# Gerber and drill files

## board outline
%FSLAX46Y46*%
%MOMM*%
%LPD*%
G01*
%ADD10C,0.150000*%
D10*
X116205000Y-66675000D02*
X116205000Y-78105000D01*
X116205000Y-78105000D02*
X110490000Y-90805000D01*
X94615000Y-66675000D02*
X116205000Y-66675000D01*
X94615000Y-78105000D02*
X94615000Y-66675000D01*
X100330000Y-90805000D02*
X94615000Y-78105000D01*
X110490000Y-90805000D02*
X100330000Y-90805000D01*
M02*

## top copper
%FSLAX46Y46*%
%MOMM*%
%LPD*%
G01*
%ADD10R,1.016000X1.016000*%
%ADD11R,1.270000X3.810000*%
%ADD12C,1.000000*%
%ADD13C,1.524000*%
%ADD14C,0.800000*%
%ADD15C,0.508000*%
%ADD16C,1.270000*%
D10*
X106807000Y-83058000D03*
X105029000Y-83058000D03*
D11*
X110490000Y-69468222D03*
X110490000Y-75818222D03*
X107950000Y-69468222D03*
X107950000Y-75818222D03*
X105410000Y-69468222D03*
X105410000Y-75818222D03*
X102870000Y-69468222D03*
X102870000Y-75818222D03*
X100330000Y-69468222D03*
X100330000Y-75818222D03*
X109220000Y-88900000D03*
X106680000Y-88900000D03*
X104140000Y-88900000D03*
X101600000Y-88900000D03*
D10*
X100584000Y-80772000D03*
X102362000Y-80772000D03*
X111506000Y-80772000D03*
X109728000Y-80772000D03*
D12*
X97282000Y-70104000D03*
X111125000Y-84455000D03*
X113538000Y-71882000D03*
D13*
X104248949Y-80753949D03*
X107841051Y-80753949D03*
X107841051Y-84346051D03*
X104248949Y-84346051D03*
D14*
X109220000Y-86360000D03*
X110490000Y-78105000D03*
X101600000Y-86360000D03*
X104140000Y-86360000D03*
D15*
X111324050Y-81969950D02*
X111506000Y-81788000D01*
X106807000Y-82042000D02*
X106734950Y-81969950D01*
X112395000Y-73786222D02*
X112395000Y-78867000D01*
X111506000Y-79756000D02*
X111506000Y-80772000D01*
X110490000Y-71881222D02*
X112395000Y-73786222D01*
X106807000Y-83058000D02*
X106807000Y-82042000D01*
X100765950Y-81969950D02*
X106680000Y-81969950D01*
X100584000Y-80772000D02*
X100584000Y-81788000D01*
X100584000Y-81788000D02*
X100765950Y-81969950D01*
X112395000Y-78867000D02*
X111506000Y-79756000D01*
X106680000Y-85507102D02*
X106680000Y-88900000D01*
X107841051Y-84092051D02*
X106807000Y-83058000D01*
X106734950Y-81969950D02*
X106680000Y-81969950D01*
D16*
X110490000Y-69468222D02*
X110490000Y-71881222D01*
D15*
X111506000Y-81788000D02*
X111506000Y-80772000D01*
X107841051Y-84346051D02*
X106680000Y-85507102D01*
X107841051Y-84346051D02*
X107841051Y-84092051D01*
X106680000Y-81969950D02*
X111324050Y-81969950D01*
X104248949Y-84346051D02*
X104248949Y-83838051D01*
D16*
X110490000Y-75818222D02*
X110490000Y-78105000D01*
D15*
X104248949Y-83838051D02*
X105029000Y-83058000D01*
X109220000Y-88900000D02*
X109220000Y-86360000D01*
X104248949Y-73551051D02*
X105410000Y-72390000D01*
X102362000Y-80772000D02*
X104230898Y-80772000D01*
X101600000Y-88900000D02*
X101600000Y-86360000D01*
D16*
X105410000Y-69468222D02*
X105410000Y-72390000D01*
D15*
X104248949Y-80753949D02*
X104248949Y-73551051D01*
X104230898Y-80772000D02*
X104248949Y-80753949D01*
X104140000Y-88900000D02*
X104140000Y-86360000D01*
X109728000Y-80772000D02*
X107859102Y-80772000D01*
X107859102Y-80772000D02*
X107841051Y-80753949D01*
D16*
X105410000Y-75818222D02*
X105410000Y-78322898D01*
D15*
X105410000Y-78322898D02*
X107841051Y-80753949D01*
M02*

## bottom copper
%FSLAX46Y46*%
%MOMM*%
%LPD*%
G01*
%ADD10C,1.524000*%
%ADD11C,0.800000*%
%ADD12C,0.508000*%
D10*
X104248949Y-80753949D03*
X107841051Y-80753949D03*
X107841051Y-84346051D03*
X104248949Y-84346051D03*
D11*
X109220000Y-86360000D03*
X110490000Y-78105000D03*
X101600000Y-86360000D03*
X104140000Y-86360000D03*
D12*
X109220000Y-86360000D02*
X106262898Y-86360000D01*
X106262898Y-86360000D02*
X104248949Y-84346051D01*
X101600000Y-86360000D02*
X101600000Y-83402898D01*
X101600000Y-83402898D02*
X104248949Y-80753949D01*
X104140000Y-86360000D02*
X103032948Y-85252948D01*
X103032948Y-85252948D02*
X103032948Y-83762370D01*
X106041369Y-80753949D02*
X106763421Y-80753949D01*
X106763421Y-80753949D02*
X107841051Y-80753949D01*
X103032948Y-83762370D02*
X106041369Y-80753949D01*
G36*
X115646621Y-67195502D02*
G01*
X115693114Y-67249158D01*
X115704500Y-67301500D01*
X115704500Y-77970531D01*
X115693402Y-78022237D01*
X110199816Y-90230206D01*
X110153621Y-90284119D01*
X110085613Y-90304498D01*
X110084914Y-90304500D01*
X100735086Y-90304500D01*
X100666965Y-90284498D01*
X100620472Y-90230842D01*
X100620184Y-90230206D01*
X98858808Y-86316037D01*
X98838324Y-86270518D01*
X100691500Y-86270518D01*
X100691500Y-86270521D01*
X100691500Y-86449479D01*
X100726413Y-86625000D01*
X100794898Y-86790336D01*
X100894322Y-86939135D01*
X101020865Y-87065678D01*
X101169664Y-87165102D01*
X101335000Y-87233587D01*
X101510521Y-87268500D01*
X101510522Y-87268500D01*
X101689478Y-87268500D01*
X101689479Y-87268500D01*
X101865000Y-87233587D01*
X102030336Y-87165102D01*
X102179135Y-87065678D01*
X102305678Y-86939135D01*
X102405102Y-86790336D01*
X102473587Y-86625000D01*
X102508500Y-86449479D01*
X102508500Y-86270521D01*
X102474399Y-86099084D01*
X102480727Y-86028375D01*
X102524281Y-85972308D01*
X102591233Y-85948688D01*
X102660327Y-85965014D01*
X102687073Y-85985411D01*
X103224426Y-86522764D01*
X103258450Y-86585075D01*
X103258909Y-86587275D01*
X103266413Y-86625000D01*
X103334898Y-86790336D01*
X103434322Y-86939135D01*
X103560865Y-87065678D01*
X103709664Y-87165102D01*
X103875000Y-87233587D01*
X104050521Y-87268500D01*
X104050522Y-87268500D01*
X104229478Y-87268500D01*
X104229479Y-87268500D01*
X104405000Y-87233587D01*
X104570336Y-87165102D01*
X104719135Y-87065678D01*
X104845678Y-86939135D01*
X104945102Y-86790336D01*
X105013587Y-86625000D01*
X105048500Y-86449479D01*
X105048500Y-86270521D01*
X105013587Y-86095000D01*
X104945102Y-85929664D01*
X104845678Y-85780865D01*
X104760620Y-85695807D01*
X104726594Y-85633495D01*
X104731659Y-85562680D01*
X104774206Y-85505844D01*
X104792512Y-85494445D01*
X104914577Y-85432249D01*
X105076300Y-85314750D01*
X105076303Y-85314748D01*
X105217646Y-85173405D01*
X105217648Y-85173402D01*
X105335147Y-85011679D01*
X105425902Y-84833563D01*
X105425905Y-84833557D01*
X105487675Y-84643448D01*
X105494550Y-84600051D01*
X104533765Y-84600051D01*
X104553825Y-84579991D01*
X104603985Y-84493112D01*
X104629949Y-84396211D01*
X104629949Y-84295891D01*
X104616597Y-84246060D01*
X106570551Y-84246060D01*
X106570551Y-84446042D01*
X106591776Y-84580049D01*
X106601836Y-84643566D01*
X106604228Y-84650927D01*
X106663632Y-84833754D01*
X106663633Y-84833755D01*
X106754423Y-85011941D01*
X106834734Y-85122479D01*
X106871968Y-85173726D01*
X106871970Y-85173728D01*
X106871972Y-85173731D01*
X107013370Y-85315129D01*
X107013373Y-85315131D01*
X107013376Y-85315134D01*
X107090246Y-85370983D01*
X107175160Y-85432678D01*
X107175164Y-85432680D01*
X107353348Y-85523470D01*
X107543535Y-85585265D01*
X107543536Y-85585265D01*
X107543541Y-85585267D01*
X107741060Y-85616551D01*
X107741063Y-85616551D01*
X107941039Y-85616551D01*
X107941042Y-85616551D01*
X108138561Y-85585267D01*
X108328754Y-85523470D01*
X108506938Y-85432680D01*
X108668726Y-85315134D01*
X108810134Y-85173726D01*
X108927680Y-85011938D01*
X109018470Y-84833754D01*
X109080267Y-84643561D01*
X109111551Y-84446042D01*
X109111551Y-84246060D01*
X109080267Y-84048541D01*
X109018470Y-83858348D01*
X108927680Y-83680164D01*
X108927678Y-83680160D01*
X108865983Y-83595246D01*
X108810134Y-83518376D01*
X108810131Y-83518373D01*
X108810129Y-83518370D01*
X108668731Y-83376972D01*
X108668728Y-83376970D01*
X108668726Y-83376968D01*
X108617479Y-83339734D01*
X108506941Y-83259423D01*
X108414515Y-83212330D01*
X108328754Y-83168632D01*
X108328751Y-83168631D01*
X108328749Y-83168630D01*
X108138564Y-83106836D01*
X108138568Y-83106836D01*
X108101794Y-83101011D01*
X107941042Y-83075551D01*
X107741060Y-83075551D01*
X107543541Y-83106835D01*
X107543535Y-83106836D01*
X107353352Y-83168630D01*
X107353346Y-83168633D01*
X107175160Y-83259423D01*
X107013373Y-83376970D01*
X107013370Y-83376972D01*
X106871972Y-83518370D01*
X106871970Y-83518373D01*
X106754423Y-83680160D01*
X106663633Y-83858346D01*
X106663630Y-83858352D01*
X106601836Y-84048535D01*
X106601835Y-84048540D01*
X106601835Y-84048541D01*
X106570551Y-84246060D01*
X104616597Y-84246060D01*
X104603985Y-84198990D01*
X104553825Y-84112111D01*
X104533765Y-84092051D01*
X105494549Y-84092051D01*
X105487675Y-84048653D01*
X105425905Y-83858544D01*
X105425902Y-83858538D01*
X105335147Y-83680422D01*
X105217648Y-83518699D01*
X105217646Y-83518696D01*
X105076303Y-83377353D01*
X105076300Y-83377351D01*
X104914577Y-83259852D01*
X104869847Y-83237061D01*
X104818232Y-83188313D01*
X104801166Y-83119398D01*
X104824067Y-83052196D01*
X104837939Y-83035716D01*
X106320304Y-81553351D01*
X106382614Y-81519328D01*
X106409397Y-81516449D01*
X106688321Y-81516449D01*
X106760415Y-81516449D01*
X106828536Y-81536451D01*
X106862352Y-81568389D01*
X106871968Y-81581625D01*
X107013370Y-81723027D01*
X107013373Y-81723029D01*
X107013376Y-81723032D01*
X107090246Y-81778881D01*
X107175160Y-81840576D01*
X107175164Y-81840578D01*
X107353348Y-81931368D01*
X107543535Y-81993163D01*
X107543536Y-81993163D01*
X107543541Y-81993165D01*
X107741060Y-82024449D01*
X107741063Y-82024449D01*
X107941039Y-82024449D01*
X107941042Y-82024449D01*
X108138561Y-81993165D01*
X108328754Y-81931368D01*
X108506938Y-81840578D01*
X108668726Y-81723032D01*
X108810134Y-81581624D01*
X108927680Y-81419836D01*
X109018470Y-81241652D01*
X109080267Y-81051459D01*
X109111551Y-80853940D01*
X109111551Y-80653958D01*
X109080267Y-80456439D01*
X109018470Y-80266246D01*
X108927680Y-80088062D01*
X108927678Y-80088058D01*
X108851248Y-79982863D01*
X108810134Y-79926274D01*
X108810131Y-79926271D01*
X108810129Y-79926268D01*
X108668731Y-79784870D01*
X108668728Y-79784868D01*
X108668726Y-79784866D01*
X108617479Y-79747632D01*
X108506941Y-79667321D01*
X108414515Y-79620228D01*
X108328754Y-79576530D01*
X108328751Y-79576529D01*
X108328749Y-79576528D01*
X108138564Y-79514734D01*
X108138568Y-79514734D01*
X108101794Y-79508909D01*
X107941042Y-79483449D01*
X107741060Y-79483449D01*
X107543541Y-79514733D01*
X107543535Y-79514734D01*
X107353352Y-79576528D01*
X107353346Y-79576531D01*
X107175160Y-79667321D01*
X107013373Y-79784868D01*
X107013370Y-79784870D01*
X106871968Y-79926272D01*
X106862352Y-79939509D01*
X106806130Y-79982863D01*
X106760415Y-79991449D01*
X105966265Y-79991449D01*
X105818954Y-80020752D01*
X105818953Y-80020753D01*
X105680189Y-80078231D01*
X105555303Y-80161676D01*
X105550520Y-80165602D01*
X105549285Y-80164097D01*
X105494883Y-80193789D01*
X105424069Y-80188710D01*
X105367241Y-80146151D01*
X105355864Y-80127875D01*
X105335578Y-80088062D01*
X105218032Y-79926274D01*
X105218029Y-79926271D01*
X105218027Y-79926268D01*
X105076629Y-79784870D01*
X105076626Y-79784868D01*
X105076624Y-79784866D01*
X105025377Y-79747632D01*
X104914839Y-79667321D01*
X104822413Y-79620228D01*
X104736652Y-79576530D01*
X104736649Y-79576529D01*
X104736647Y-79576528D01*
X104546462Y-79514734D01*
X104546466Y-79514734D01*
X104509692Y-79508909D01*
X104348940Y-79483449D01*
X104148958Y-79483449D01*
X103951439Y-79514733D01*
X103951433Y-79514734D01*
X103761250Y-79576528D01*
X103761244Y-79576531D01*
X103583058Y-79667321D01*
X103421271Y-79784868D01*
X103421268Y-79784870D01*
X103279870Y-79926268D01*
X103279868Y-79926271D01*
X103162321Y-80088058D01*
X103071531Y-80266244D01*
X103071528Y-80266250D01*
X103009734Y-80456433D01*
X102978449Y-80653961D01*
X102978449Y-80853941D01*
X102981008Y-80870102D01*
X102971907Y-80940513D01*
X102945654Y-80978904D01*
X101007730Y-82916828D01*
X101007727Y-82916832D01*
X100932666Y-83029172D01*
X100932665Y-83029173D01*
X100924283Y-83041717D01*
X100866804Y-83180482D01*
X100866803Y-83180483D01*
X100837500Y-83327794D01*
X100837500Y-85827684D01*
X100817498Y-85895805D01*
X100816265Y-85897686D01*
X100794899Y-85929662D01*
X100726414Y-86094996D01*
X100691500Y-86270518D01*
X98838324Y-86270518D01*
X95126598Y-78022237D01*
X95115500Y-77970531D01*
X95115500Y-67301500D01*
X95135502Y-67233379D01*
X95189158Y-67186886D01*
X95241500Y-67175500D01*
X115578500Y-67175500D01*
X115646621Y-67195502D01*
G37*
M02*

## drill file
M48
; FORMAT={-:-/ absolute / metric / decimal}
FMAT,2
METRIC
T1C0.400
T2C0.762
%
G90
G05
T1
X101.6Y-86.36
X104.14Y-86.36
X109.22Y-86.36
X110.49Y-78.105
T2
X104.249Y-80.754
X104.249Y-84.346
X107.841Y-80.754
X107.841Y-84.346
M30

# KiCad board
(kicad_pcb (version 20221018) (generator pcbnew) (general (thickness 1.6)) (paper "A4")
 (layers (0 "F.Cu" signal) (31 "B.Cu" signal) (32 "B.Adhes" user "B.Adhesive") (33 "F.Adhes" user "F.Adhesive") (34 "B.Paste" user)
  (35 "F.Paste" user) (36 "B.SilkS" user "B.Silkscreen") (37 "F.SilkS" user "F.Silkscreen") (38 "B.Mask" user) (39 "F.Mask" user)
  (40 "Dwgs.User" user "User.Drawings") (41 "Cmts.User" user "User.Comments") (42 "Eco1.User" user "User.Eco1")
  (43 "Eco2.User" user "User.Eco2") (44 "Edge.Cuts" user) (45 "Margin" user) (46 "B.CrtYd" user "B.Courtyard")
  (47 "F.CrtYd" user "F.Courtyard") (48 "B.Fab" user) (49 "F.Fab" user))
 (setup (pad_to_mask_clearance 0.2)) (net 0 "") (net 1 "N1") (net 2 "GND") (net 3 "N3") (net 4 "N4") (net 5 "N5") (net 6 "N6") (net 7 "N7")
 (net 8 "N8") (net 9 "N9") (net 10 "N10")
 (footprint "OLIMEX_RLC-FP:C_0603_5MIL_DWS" (layer "F.Cu") (at 105.918 83.058 180)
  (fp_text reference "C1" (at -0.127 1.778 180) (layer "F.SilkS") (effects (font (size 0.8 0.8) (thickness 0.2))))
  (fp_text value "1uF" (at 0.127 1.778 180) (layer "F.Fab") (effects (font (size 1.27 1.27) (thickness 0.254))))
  (pad "1" smd rect (at -0.889 0 180) (size 1.016 1.016) (layers "F.Cu" "F.Paste" "F.Mask") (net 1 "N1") (solder_mask_margin 0.0508)
   (clearance 0.0508))
  (pad "2" smd rect (at 0.889 0 180) (size 1.016 1.016) (layers "F.Cu" "F.Paste" "F.Mask") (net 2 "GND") (solder_mask_margin 0.0508)
   (clearance 0.0508)))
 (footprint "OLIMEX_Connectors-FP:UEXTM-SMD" (layer "F.Cu") (at 105.41 72.643222)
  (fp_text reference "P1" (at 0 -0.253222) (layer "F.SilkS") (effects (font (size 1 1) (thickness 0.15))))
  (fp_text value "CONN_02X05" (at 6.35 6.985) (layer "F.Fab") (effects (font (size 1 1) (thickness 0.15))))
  (pad "1" smd rect (at 5.08 -3.175) (size 1.27 3.81) (layers "F.Cu" "F.Paste" "F.Mask") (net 1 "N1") (solder_mask_margin 0.0508)
   (solder_paste_margin -0.0508) (clearance 0.0508))
  (pad "2" smd rect (at 5.08 3.175) (size 1.27 3.81) (layers "F.Cu" "F.Paste" "F.Mask") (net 2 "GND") (solder_mask_margin 0.0508)
   (solder_paste_margin -0.0508) (clearance 0.0508))
  (pad "3" smd rect (at 2.54 -3.175) (size 1.27 3.81) (layers "F.Cu" "F.Paste" "F.Mask") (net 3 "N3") (solder_mask_margin 0.0508)
   (solder_paste_margin -0.0508) (clearance 0.0508))
  (pad "4" smd rect (at 2.54 3.175) (size 1.27 3.81) (layers "F.Cu" "F.Paste" "F.Mask") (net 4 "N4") (solder_mask_margin 0.0508)
   (solder_paste_margin -0.0508) (clearance 0.0508))
  (pad "5" smd rect (at 0 -3.175) (size 1.27 3.81) (layers "F.Cu" "F.Paste" "F.Mask") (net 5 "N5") (solder_mask_margin 0.0508)
   (solder_paste_margin -0.0508) (clearance 0.0508))
  (pad "6" smd rect (at 0 3.175) (size 1.27 3.81) (layers "F.Cu" "F.Paste" "F.Mask") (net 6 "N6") (solder_mask_margin 0.0508)
   (solder_paste_margin -0.0508) (clearance 0.0508))
  (pad "7" smd rect (at -2.54 -3.175) (size 1.27 3.81) (layers "F.Cu" "F.Paste" "F.Mask") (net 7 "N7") (solder_mask_margin 0.0508)
   (solder_paste_margin -0.0508) (clearance 0.0508))
  (pad "8" smd rect (at -2.54 3.175) (size 1.27 3.81) (layers "F.Cu" "F.Paste" "F.Mask") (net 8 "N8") (solder_mask_margin 0.0508)
   (solder_paste_margin -0.0508) (clearance 0.0508))
  (pad "9" smd rect (at -5.08 -3.175) (size 1.27 3.81) (layers "F.Cu" "F.Paste" "F.Mask") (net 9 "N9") (solder_mask_margin 0.0508)
   (solder_paste_margin -0.0508) (clearance 0.0508))
  (pad "10" smd rect (at -5.08 3.175) (size 1.27 3.81) (layers "F.Cu" "F.Paste" "F.Mask") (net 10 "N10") (solder_mask_margin 0.0508)
   (solder_paste_margin -0.0508) (clearance 0.0508)))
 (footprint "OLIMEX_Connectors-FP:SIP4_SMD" (layer "F.Cu") (at 105.41 88.9 180)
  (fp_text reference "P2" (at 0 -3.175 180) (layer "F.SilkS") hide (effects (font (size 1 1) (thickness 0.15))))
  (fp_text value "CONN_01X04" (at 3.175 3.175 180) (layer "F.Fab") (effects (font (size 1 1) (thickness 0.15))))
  (pad "1" smd rect (at -3.81 0 180) (size 1.27 3.81) (layers "F.Cu" "F.Mask") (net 2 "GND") (solder_mask_margin 0.0508)
   (solder_paste_margin -0.0508) (clearance 0.0508))
  (pad "2" smd rect (at -1.27 0 180) (size 1.27 3.81) (layers "F.Cu" "F.Mask") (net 1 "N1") (solder_mask_margin 0.0508)
   (solder_paste_margin -0.0508) (clearance 0.0508))
  (pad "3" smd rect (at 1.27 0 180) (size 1.27 3.81) (layers "F.Cu" "F.Mask") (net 6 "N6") (solder_mask_margin 0.0508)
   (solder_paste_margin -0.0508) (clearance 0.0508))
  (pad "4" smd rect (at 3.81 0 180) (size 1.27 3.81) (layers "F.Cu" "F.Mask") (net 5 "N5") (solder_mask_margin 0.0508)
   (solder_paste_margin -0.0508) (clearance 0.0508)))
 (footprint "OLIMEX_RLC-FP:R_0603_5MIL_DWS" (layer "F.Cu") (at 101.473 80.772)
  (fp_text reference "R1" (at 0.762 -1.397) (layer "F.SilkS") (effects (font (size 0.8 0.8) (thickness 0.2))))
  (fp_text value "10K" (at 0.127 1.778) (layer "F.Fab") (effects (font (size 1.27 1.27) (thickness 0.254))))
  (pad "1" smd rect (at -0.889 0) (size 1.016 1.016) (layers "F.Cu" "F.Paste" "F.Mask") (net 1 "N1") (solder_mask_margin 0.0508))
  (pad "2" smd rect (at 0.889 0) (size 1.016 1.016) (layers "F.Cu" "F.Paste" "F.Mask") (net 5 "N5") (solder_mask_margin 0.0508)))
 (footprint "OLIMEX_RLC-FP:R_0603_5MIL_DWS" (layer "F.Cu") (at 110.617 80.772 180)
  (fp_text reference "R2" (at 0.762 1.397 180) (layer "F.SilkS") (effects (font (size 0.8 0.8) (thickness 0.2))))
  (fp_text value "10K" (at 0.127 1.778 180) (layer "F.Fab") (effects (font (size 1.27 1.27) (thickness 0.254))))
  (pad "1" smd rect (at -0.889 0 180) (size 1.016 1.016) (layers "F.Cu" "F.Paste" "F.Mask") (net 1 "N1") (solder_mask_margin 0.0508))
  (pad "2" smd rect (at 0.889 0 180) (size 1.016 1.016) (layers "F.Cu" "F.Paste" "F.Mask") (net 6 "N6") (solder_mask_margin 0.0508)))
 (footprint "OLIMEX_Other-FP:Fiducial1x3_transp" (layer "F.Cu") (at 97.282 70.104)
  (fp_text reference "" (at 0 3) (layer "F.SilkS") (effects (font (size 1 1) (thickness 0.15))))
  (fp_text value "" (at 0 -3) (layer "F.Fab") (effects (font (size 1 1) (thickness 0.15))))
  (pad "Fid1" connect circle (at 0 0) (size 1 1) (layers "F.Cu" "F.Mask") (solder_mask_margin 0.127) (clearance 1.016) (zone_connect 0)))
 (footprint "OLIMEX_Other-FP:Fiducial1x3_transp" (layer "F.Cu") (at 111.125 84.455)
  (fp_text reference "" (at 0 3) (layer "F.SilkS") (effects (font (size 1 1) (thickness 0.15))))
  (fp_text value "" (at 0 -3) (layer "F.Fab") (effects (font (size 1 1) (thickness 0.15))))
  (pad "Fid1" connect circle (at 0 0) (size 1 1) (layers "F.Cu" "F.Mask") (solder_mask_margin 0.127) (clearance 1.016) (zone_connect 0)))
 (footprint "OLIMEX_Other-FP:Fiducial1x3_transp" (layer "F.Cu") (at 113.538 71.882)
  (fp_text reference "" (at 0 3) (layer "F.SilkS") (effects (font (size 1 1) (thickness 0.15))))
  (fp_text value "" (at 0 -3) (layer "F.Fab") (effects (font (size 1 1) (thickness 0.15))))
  (pad "Fid1" connect circle (at 0 0) (size 1 1) (layers "F.Cu" "F.Mask") (solder_mask_margin 0.127) (clearance 1.016) (zone_connect 0)))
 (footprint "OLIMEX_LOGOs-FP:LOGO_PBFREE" (layer "F.Cu") (at 98.044 80.01)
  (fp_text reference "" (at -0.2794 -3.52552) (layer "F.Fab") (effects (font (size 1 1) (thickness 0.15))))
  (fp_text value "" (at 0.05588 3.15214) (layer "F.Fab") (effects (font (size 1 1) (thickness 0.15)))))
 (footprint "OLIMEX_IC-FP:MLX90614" (layer "B.Cu") (at 106.045 82.55 -135)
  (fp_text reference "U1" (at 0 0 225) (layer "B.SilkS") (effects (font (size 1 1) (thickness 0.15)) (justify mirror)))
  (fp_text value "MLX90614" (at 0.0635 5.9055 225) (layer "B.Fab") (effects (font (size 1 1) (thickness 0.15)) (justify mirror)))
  (pad "1" thru_hole circle (at 0 2.54 225) (size 1.524 1.524) (drill 0.762) (layers "*.Cu" "*.Mask") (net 5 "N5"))
  (pad "2" thru_hole circle (at -2.54 0 225) (size 1.524 1.524) (drill 0.762) (layers "*.Cu" "*.Mask") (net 6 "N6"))
  (pad "3" thru_hole circle (at 0 -2.54 225) (size 1.524 1.524) (drill 0.762) (layers "*.Cu" "*.Mask") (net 1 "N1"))
  (pad "4" thru_hole circle (at 2.54 0 225) (size 1.524 1.524) (drill 0.762) (layers "*.Cu" "*.Mask") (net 2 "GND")))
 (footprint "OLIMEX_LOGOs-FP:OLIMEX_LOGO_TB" (layer "B.Cu") (at 105.41 69.85 180)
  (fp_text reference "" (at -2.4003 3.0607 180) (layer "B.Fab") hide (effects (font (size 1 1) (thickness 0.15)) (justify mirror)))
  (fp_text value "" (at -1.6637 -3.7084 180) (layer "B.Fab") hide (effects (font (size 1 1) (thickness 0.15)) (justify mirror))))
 (gr_line (start 116.205 66.675) (end 116.205 78.105) (stroke (width 0.15) (type solid)) (layer "Edge.Cuts"))
 (gr_line (start 116.205 78.105) (end 110.49 90.805) (stroke (width 0.15) (type solid)) (layer "Edge.Cuts"))
 (gr_line (start 94.615 66.675) (end 116.205 66.675) (stroke (width 0.15) (type solid)) (layer "Edge.Cuts"))
 (gr_line (start 94.615 78.105) (end 94.615 66.675) (stroke (width 0.15) (type solid)) (layer "Edge.Cuts"))
 (gr_line (start 100.33 90.805) (end 94.615 78.105) (stroke (width 0.15) (type solid)) (layer "Edge.Cuts"))
 (gr_line (start 110.49 90.805) (end 100.33 90.805) (stroke (width 0.15) (type solid)) (layer "Edge.Cuts"))
 (segment (start 111.32405 81.96995) (end 111.506 81.788) (width 0.508) (layer "F.Cu") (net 1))
 (segment (start 106.807 82.042) (end 106.73495 81.96995) (width 0.508) (layer "F.Cu") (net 1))
 (segment (start 112.395 73.786222) (end 112.395 78.867) (width 0.508) (layer "F.Cu") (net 1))
 (segment (start 111.506 79.756) (end 111.506 80.772) (width 0.508) (layer "F.Cu") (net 1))
 (segment (start 110.49 71.881222) (end 112.395 73.786222) (width 0.508) (layer "F.Cu") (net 1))
 (segment (start 106.807 83.058) (end 106.807 82.042) (width 0.508) (layer "F.Cu") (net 1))
 (segment (start 100.76595 81.96995) (end 106.68 81.96995) (width 0.508) (layer "F.Cu") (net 1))
 (segment (start 100.584 80.772) (end 100.584 81.788) (width 0.508) (layer "F.Cu") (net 1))
 (segment (start 100.584 81.788) (end 100.76595 81.96995) (width 0.508) (layer "F.Cu") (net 1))
 (segment (start 112.395 78.867) (end 111.506 79.756) (width 0.508) (layer "F.Cu") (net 1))
 (segment (start 106.68 85.507102) (end 106.68 88.9) (width 0.508) (layer "F.Cu") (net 1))
 (segment (start 107.841051 84.092051) (end 106.807 83.058) (width 0.508) (layer "F.Cu") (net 1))
 (segment (start 106.73495 81.96995) (end 106.68 81.96995) (width 0.508) (layer "F.Cu") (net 1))
 (segment (start 110.49 69.468222) (end 110.49 71.881222) (width 1.27) (layer "F.Cu") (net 1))
 (segment (start 111.506 81.788) (end 111.506 80.772) (width 0.508) (layer "F.Cu") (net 1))
 (segment (start 107.841051 84.346051) (end 106.68 85.507102) (width 0.508) (layer "F.Cu") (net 1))
 (segment (start 107.841051 84.346051) (end 107.841051 84.092051) (width 0.508) (layer "F.Cu") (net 1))
 (segment (start 106.68 81.96995) (end 111.32405 81.96995) (width 0.508) (layer "F.Cu") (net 1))
 (segment (start 104.248949 84.346051) (end 104.248949 83.838051) (width 0.508) (layer "F.Cu") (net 2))
 (segment (start 110.49 75.818222) (end 110.49 78.105) (width 1.27) (layer "F.Cu") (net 2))
 (segment (start 104.248949 83.838051) (end 105.029 83.058) (width 0.508) (layer "F.Cu") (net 2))
 (segment (start 109.22 88.9) (end 109.22 86.36) (width 0.508) (layer "F.Cu") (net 2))
 (via (at 109.22 86.36) (size 0.8) (drill 0.4) (layers "F.Cu" "B.Cu") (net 2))
 (via (at 110.49 78.105) (size 0.8) (drill 0.4) (layers "F.Cu" "B.Cu") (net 2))
 (segment (start 109.22 86.36) (end 106.262898 86.36) (width 0.508) (layer "B.Cu") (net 2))
 (segment (start 106.262898 86.36) (end 104.248949 84.346051) (width 0.508) (layer "B.Cu") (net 2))
 (segment (start 104.248949 73.551051) (end 105.41 72.39) (width 0.508) (layer "F.Cu") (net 5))
 (segment (start 102.362 80.772) (end 104.230898 80.772) (width 0.508) (layer "F.Cu") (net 5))
 (segment (start 101.6 88.9) (end 101.6 86.36) (width 0.508) (layer "F.Cu") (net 5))
 (segment (start 105.41 69.468222) (end 105.41 72.39) (width 1.27) (layer "F.Cu") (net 5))
 (segment (start 104.248949 80.753949) (end 104.248949 73.551051) (width 0.508) (layer "F.Cu") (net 5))
 (segment (start 104.230898 80.772) (end 104.248949 80.753949) (width 0.508) (layer "F.Cu") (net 5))
 (via (at 101.6 86.36) (size 0.8) (drill 0.4) (layers "F.Cu" "B.Cu") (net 5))
 (segment (start 101.6 86.36) (end 101.6 83.402898) (width 0.508) (layer "B.Cu") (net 5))
 (segment (start 101.6 83.402898) (end 104.248949 80.753949) (width 0.508) (layer "B.Cu") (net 5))
 (segment (start 104.14 88.9) (end 104.14 86.36) (width 0.508) (layer "F.Cu") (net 6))
 (segment (start 109.728 80.772) (end 107.859102 80.772) (width 0.508) (layer "F.Cu") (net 6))
 (segment (start 107.859102 80.772) (end 107.841051 80.753949) (width 0.508) (layer "F.Cu") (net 6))
 (segment (start 105.41 75.818222) (end 105.41 78.322898) (width 1.27) (layer "F.Cu") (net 6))
 (segment (start 105.41 78.322898) (end 107.841051 80.753949) (width 0.508) (layer "F.Cu") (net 6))
 (via (at 104.14 86.36) (size 0.8) (drill 0.4) (layers "F.Cu" "B.Cu") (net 6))
 (segment (start 104.14 86.36) (end 103.032948 85.252948) (width 0.508) (layer "B.Cu") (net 6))
 (segment (start 103.032948 85.252948) (end 103.032948 83.76237) (width 0.508) (layer "B.Cu") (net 6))
 (segment (start 106.041369 80.753949) (end 106.763421 80.753949) (width 0.508) (layer "B.Cu") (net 6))
 (segment (start 106.763421 80.753949) (end 107.841051 80.753949) (width 0.508) (layer "B.Cu") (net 6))
 (segment (start 103.032948 83.76237) (end 106.041369 80.753949) (width 0.508) (layer "B.Cu") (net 6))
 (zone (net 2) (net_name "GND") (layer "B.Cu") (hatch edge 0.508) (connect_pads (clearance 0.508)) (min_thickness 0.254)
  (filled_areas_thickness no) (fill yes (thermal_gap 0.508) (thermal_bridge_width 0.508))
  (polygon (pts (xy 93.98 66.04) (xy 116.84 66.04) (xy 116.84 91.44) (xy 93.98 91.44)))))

